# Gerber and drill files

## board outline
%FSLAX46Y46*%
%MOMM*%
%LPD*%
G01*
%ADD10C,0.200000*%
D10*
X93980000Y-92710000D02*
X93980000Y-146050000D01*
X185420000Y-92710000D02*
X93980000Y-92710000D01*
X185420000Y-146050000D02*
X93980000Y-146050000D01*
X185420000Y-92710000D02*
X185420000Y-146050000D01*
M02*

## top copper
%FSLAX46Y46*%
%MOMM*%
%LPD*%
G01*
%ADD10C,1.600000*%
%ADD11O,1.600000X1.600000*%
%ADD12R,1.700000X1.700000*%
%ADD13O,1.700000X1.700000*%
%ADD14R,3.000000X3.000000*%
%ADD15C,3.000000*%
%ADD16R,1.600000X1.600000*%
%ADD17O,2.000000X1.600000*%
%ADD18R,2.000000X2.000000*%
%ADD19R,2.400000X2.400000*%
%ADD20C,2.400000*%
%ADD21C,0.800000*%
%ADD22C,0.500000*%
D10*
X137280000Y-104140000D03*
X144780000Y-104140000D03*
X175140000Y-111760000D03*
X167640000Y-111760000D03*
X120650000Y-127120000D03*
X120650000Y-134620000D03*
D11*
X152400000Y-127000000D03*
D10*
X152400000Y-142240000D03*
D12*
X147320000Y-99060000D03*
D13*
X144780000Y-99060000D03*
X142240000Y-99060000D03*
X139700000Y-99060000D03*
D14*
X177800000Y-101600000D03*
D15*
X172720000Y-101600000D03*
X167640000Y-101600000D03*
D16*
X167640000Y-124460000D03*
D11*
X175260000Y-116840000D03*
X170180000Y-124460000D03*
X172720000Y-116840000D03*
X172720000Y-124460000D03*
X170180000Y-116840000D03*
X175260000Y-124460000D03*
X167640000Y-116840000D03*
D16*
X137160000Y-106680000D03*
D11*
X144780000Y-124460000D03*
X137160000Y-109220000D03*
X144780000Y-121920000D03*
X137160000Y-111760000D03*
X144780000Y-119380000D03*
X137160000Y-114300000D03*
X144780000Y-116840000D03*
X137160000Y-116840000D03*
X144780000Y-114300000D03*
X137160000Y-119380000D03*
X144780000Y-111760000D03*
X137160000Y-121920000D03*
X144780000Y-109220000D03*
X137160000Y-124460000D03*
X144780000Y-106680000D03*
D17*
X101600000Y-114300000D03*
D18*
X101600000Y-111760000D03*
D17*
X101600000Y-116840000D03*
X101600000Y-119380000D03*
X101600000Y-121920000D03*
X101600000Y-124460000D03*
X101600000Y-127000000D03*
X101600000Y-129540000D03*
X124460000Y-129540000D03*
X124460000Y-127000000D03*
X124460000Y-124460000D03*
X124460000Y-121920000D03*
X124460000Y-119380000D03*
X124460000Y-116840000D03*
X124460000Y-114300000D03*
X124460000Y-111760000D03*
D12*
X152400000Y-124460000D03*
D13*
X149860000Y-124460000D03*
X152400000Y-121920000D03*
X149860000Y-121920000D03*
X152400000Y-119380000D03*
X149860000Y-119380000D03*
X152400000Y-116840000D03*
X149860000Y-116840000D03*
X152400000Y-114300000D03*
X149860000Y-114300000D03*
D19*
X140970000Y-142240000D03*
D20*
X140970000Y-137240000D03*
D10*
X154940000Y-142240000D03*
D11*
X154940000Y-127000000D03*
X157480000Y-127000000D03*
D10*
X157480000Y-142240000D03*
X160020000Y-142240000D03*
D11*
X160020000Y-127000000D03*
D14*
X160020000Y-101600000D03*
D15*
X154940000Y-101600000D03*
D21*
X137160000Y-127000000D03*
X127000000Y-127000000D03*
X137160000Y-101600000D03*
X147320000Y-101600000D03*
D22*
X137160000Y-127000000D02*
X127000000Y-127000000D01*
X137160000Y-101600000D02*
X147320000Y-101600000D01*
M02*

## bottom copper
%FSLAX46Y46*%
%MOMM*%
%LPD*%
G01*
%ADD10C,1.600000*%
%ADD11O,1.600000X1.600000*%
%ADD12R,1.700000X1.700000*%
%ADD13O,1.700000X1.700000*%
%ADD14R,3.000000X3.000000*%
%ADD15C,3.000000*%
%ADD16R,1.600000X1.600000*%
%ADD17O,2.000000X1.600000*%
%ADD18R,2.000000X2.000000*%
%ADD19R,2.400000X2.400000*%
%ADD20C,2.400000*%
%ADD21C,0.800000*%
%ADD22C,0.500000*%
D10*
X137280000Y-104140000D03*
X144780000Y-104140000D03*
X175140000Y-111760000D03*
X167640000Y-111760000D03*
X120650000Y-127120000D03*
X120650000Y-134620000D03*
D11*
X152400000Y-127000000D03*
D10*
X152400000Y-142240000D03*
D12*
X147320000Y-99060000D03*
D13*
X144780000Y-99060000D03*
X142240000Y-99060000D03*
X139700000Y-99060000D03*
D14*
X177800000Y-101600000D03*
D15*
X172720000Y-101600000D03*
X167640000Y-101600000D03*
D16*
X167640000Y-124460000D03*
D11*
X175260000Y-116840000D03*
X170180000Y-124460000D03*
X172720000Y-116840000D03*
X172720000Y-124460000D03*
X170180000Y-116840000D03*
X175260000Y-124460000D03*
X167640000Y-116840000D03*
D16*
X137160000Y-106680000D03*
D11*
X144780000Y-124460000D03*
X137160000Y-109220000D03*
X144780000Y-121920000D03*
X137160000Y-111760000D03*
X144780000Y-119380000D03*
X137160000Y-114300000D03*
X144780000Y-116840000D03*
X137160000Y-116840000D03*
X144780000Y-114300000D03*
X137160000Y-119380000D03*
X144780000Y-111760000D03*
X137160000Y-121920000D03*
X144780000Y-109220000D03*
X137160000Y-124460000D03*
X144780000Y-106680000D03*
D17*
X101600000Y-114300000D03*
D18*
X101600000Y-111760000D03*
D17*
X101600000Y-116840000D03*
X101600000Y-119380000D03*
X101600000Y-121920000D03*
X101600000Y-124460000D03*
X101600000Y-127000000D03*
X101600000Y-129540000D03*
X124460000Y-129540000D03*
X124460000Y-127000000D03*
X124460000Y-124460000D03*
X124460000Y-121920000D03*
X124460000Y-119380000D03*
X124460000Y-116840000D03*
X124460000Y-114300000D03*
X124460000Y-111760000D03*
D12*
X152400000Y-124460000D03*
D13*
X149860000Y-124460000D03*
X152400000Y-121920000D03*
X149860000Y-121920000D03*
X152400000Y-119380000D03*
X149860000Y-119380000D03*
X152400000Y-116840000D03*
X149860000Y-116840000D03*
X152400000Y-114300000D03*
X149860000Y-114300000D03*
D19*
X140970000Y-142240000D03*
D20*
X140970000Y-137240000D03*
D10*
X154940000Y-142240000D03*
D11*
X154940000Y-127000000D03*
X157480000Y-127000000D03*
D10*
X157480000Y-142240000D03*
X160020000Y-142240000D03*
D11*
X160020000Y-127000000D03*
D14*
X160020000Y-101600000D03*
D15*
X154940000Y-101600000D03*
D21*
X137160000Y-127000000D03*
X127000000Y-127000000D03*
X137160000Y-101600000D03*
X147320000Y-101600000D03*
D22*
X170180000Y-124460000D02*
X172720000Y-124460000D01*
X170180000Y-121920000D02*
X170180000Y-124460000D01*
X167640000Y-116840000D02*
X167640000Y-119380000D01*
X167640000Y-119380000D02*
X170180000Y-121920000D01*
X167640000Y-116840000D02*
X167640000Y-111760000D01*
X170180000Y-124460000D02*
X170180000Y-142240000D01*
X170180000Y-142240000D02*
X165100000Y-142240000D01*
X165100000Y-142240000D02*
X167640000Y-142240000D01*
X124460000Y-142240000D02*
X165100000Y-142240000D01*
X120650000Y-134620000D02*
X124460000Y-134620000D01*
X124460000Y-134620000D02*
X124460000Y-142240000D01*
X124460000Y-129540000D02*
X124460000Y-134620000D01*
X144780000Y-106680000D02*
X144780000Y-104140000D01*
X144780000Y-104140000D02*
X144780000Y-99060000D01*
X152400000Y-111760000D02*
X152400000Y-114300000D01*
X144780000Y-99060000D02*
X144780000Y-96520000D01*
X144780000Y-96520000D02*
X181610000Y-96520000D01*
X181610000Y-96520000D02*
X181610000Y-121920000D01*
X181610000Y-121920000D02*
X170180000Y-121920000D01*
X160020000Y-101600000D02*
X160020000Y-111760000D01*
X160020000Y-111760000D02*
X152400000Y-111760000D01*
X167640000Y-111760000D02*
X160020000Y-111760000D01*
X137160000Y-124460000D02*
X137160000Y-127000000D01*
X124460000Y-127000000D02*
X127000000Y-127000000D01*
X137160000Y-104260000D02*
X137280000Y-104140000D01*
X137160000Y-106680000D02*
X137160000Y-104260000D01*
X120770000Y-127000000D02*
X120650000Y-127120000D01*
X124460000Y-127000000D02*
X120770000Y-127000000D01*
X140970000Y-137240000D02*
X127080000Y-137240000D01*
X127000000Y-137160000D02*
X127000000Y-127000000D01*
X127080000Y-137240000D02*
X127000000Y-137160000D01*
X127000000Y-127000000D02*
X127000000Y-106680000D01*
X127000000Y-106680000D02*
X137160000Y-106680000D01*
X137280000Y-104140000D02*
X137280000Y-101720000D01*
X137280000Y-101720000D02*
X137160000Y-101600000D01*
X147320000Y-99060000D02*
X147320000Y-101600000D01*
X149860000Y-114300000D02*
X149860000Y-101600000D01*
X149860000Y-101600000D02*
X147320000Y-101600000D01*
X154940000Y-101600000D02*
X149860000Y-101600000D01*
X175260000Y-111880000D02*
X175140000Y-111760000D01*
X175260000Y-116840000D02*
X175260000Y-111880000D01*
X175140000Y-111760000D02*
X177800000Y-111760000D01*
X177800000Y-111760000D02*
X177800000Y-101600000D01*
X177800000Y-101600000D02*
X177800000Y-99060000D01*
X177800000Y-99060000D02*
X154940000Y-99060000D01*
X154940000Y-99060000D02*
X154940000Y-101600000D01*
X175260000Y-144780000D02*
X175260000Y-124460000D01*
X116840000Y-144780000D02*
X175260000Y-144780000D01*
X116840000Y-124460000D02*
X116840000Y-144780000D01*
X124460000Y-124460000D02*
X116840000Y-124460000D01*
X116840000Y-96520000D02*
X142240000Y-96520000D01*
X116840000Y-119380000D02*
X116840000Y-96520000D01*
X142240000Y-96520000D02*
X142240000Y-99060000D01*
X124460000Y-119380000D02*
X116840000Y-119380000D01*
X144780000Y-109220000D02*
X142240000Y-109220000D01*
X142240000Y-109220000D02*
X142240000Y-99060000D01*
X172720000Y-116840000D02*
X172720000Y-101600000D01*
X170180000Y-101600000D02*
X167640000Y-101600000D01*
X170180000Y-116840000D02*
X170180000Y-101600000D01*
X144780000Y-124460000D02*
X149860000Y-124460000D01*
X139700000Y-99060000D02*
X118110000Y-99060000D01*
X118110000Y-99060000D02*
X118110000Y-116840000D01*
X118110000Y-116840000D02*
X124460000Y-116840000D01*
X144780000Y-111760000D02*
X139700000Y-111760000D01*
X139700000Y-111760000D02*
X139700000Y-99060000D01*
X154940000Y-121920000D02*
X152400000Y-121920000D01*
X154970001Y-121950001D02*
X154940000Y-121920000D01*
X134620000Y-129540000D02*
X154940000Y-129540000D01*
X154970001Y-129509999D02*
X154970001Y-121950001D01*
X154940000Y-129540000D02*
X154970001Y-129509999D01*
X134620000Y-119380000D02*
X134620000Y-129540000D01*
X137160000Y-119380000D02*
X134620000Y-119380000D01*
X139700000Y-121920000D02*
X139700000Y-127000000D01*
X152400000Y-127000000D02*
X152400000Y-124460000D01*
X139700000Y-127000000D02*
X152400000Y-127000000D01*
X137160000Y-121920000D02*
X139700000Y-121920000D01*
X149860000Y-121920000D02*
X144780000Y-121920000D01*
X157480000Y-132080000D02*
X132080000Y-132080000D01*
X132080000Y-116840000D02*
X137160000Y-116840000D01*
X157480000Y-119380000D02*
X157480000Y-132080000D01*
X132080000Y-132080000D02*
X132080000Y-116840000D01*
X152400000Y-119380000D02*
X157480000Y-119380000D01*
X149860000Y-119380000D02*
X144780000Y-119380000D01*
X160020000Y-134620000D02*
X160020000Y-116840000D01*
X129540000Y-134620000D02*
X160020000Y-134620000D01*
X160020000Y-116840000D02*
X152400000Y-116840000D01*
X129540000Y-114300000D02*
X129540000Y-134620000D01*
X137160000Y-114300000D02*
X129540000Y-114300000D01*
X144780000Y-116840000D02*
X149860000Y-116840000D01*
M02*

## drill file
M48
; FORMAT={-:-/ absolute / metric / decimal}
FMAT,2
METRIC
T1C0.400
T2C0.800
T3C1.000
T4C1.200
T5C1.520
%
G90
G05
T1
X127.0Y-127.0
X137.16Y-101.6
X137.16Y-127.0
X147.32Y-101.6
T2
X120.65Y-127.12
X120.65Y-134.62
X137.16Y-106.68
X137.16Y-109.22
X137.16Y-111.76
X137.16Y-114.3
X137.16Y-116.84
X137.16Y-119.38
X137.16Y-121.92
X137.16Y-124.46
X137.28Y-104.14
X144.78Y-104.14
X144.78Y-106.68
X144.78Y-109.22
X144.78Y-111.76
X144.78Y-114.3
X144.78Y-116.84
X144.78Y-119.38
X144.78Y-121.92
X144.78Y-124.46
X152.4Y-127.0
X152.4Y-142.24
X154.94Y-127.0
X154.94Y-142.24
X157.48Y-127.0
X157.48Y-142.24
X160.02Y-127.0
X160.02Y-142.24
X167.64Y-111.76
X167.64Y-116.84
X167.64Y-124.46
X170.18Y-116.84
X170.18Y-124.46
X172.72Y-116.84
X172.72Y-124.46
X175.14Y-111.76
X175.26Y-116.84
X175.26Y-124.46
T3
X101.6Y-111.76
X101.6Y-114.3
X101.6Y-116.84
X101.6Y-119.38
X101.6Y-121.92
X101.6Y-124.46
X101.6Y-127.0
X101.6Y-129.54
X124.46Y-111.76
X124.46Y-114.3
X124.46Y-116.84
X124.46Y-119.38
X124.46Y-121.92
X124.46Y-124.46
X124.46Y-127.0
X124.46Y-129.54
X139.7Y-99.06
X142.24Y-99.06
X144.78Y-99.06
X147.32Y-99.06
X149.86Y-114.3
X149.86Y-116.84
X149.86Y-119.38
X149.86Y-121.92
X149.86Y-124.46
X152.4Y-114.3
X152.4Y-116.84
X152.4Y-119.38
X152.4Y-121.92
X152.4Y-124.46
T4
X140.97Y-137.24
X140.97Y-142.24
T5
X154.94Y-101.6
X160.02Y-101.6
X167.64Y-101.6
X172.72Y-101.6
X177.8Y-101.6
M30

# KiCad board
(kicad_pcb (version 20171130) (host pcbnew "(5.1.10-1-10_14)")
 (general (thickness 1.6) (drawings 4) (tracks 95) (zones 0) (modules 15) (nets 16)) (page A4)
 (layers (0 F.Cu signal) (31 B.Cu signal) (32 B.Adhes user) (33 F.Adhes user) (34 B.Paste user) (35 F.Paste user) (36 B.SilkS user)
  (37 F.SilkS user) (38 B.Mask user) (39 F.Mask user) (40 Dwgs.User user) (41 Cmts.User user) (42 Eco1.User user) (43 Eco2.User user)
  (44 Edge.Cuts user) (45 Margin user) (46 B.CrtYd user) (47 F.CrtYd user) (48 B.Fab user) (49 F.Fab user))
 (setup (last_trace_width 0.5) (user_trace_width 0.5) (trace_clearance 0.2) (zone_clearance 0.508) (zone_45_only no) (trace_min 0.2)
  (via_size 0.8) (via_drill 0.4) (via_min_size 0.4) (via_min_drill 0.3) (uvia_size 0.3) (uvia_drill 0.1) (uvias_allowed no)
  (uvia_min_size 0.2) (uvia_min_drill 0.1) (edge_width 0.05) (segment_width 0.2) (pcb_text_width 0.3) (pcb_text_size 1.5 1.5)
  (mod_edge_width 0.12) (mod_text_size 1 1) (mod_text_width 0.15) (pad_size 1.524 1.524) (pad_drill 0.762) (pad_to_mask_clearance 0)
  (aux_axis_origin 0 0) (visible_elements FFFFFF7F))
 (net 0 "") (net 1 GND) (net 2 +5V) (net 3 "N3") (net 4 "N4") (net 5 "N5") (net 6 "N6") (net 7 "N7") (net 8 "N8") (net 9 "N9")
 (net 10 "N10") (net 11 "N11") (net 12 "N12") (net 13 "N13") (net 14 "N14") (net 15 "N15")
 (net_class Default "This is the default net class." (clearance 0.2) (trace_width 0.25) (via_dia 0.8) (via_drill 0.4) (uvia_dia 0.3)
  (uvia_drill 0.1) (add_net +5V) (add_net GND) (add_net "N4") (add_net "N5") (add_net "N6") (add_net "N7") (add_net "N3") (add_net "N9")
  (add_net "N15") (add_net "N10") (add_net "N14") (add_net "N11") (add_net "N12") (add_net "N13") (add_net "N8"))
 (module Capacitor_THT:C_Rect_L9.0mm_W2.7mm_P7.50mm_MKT (layer F.Cu) (at 144.78 104.14 180)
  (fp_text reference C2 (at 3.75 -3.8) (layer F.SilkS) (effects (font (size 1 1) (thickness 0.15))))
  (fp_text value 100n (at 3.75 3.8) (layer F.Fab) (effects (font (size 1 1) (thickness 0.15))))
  (pad 2 thru_hole circle (at 7.5 0 180) (size 1.6 1.6) (drill 0.8) (layers *.Cu *.Mask) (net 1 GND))
  (pad 1 thru_hole circle (at 0 0 180) (size 1.6 1.6) (drill 0.8) (layers *.Cu *.Mask) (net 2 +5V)))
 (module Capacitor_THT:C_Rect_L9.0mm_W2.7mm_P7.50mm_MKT (layer F.Cu) (at 167.64 111.76)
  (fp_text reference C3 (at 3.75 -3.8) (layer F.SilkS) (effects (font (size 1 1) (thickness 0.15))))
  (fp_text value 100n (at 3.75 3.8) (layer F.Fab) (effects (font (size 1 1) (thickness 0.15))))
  (pad 2 thru_hole circle (at 7.5 0) (size 1.6 1.6) (drill 0.8) (layers *.Cu *.Mask) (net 1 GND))
  (pad 1 thru_hole circle (at 0 0) (size 1.6 1.6) (drill 0.8) (layers *.Cu *.Mask) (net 2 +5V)))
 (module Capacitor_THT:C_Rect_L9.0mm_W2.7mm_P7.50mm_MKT (layer F.Cu) (at 120.65 134.62 90)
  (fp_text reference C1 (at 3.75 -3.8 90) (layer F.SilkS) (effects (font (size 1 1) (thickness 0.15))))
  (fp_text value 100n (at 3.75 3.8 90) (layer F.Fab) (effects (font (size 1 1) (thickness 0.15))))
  (pad 2 thru_hole circle (at 7.5 0 90) (size 1.6 1.6) (drill 0.8) (layers *.Cu *.Mask) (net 1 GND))
  (pad 1 thru_hole circle (at 0 0 90) (size 1.6 1.6) (drill 0.8) (layers *.Cu *.Mask) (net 2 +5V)))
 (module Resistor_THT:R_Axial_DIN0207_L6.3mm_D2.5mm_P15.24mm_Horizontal (layer F.Cu) (at 152.4 142.24 90)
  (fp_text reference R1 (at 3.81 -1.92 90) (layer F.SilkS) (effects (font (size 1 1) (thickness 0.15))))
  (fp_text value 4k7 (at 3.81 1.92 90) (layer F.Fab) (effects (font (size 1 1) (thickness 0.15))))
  (pad 2 thru_hole oval (at 15.24 0 90) (size 1.6 1.6) (drill 0.8) (layers *.Cu *.Mask) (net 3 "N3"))
  (pad 1 thru_hole circle (at 0 0 90) (size 1.6 1.6) (drill 0.8) (layers *.Cu *.Mask) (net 2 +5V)))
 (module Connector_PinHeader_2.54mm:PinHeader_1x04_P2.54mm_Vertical (layer F.Cu) (at 147.32 99.06 270)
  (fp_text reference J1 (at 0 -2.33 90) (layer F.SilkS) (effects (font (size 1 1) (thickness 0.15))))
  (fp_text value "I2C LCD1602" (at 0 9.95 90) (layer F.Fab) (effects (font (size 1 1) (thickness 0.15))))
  (pad 1 thru_hole rect (at 0 0 270) (size 1.7 1.7) (drill 1) (layers *.Cu *.Mask) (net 1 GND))
  (pad 2 thru_hole oval (at 0 2.54 270) (size 1.7 1.7) (drill 1) (layers *.Cu *.Mask) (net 2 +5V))
  (pad 3 thru_hole oval (at 0 5.08 270) (size 1.7 1.7) (drill 1) (layers *.Cu *.Mask) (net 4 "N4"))
  (pad 4 thru_hole oval (at 0 7.62 270) (size 1.7 1.7) (drill 1) (layers *.Cu *.Mask) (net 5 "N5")))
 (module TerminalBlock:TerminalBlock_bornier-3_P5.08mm (layer F.Cu) (at 177.8 101.6 180)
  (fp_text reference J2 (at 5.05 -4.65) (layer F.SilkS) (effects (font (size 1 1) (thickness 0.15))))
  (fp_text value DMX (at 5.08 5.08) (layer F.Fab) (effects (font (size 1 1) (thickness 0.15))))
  (pad 1 thru_hole rect (at 0 0 180) (size 3 3) (drill 1.52) (layers *.Cu *.Mask) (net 1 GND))
  (pad 2 thru_hole circle (at 5.08 0 180) (size 3 3) (drill 1.52) (layers *.Cu *.Mask) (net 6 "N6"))
  (pad 3 thru_hole circle (at 10.16 0 180) (size 3 3) (drill 1.52) (layers *.Cu *.Mask) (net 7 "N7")))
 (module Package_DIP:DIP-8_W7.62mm (layer F.Cu) (at 167.64 124.46 90)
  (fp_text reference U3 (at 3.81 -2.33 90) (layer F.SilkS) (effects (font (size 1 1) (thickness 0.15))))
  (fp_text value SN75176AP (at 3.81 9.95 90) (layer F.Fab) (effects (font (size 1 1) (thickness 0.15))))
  (pad 1 thru_hole rect (at 0 0 90) (size 1.6 1.6) (drill 0.8) (layers *.Cu *.Mask))
  (pad 5 thru_hole oval (at 7.62 7.62 90) (size 1.6 1.6) (drill 0.8) (layers *.Cu *.Mask) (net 1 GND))
  (pad 2 thru_hole oval (at 0 2.54 90) (size 1.6 1.6) (drill 0.8) (layers *.Cu *.Mask) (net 2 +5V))
  (pad 6 thru_hole oval (at 7.62 5.08 90) (size 1.6 1.6) (drill 0.8) (layers *.Cu *.Mask) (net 6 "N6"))
  (pad 3 thru_hole oval (at 0 5.08 90) (size 1.6 1.6) (drill 0.8) (layers *.Cu *.Mask) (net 2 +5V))
  (pad 7 thru_hole oval (at 7.62 2.54 90) (size 1.6 1.6) (drill 0.8) (layers *.Cu *.Mask) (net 7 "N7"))
  (pad 4 thru_hole oval (at 0 7.62 90) (size 1.6 1.6) (drill 0.8) (layers *.Cu *.Mask) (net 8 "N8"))
  (pad 8 thru_hole oval (at 7.62 0 90) (size 1.6 1.6) (drill 0.8) (layers *.Cu *.Mask) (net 2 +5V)))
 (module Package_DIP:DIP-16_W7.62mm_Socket (layer F.Cu) (at 137.16 106.68)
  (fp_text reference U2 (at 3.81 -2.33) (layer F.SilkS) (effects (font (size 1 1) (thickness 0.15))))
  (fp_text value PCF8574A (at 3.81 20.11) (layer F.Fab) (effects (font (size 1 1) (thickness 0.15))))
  (pad 1 thru_hole rect (at 0 0) (size 1.6 1.6) (drill 0.8) (layers *.Cu *.Mask) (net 1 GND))
  (pad 9 thru_hole oval (at 7.62 17.78) (size 1.6 1.6) (drill 0.8) (layers *.Cu *.Mask) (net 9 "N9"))
  (pad 2 thru_hole oval (at 0 2.54) (size 1.6 1.6) (drill 0.8) (layers *.Cu *.Mask))
  (pad 10 thru_hole oval (at 7.62 15.24) (size 1.6 1.6) (drill 0.8) (layers *.Cu *.Mask) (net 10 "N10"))
  (pad 3 thru_hole oval (at 0 5.08) (size 1.6 1.6) (drill 0.8) (layers *.Cu *.Mask))
  (pad 11 thru_hole oval (at 7.62 12.7) (size 1.6 1.6) (drill 0.8) (layers *.Cu *.Mask) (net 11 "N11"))
  (pad 4 thru_hole oval (at 0 7.62) (size 1.6 1.6) (drill 0.8) (layers *.Cu *.Mask) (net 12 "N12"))
  (pad 12 thru_hole oval (at 7.62 10.16) (size 1.6 1.6) (drill 0.8) (layers *.Cu *.Mask) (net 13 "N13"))
  (pad 5 thru_hole oval (at 0 10.16) (size 1.6 1.6) (drill 0.8) (layers *.Cu *.Mask) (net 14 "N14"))
  (pad 13 thru_hole oval (at 7.62 7.62) (size 1.6 1.6) (drill 0.8) (layers *.Cu *.Mask))
  (pad 6 thru_hole oval (at 0 12.7) (size 1.6 1.6) (drill 0.8) (layers *.Cu *.Mask) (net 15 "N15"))
  (pad 14 thru_hole oval (at 7.62 5.08) (size 1.6 1.6) (drill 0.8) (layers *.Cu *.Mask) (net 5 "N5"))
  (pad 7 thru_hole oval (at 0 15.24) (size 1.6 1.6) (drill 0.8) (layers *.Cu *.Mask) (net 3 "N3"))
  (pad 15 thru_hole oval (at 7.62 2.54) (size 1.6 1.6) (drill 0.8) (layers *.Cu *.Mask) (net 4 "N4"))
  (pad 8 thru_hole oval (at 0 17.78) (size 1.6 1.6) (drill 0.8) (layers *.Cu *.Mask) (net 1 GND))
  (pad 16 thru_hole oval (at 7.62 0) (size 1.6 1.6) (drill 0.8) (layers *.Cu *.Mask) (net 2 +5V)))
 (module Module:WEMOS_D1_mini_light (layer F.Cu) (at 101.6 111.76)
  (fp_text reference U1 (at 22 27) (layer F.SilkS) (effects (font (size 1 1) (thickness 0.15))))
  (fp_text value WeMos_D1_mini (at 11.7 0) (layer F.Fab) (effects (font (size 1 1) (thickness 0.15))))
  (pad 2 thru_hole oval (at 0 2.54) (size 2 1.6) (drill 1) (layers *.Cu *.Mask))
  (pad 1 thru_hole rect (at 0 0) (size 2 2) (drill 1) (layers *.Cu *.Mask))
  (pad 3 thru_hole oval (at 0 5.08) (size 2 1.6) (drill 1) (layers *.Cu *.Mask))
  (pad 4 thru_hole oval (at 0 7.62) (size 2 1.6) (drill 1) (layers *.Cu *.Mask))
  (pad 5 thru_hole oval (at 0 10.16) (size 2 1.6) (drill 1) (layers *.Cu *.Mask))
  (pad 6 thru_hole oval (at 0 12.7) (size 2 1.6) (drill 1) (layers *.Cu *.Mask))
  (pad 7 thru_hole oval (at 0 15.24) (size 2 1.6) (drill 1) (layers *.Cu *.Mask))
  (pad 8 thru_hole oval (at 0 17.78) (size 2 1.6) (drill 1) (layers *.Cu *.Mask))
  (pad 9 thru_hole oval (at 22.86 17.78) (size 2 1.6) (drill 1) (layers *.Cu *.Mask) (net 2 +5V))
  (pad 10 thru_hole oval (at 22.86 15.24) (size 2 1.6) (drill 1) (layers *.Cu *.Mask) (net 1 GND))
  (pad 11 thru_hole oval (at 22.86 12.7) (size 2 1.6) (drill 1) (layers *.Cu *.Mask) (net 8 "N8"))
  (pad 12 thru_hole oval (at 22.86 10.16) (size 2 1.6) (drill 1) (layers *.Cu *.Mask))
  (pad 13 thru_hole oval (at 22.86 7.62) (size 2 1.6) (drill 1) (layers *.Cu *.Mask) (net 4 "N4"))
  (pad 14 thru_hole oval (at 22.86 5.08) (size 2 1.6) (drill 1) (layers *.Cu *.Mask) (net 5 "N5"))
  (pad 15 thru_hole oval (at 22.86 2.54) (size 2 1.6) (drill 1) (layers *.Cu *.Mask))
  (pad 16 thru_hole oval (at 22.86 0) (size 2 1.6) (drill 1) (layers *.Cu *.Mask)))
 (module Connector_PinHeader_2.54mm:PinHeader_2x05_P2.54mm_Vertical (layer F.Cu) (at 152.4 124.46 180)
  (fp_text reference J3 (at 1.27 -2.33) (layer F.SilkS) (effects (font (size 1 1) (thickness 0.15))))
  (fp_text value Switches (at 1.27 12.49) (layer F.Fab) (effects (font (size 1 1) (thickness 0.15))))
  (pad 1 thru_hole rect (at 0 0 180) (size 1.7 1.7) (drill 1) (layers *.Cu *.Mask) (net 3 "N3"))
  (pad 2 thru_hole oval (at 2.54 0 180) (size 1.7 1.7) (drill 1) (layers *.Cu *.Mask) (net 9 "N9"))
  (pad 3 thru_hole oval (at 0 2.54 180) (size 1.7 1.7) (drill 1) (layers *.Cu *.Mask) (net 15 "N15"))
  (pad 4 thru_hole oval (at 2.54 2.54 180) (size 1.7 1.7) (drill 1) (layers *.Cu *.Mask) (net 10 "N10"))
  (pad 5 thru_hole oval (at 0 5.08 180) (size 1.7 1.7) (drill 1) (layers *.Cu *.Mask) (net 14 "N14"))
  (pad 6 thru_hole oval (at 2.54 5.08 180) (size 1.7 1.7) (drill 1) (layers *.Cu *.Mask) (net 11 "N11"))
  (pad 7 thru_hole oval (at 0 7.62 180) (size 1.7 1.7) (drill 1) (layers *.Cu *.Mask) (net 12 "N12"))
  (pad 8 thru_hole oval (at 2.54 7.62 180) (size 1.7 1.7) (drill 1) (layers *.Cu *.Mask) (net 13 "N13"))
  (pad 9 thru_hole oval (at 0 10.16 180) (size 1.7 1.7) (drill 1) (layers *.Cu *.Mask) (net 2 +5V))
  (pad 10 thru_hole oval (at 2.54 10.16 180) (size 1.7 1.7) (drill 1) (layers *.Cu *.Mask) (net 1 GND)))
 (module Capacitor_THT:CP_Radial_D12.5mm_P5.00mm (layer F.Cu) (at 140.97 142.24 90)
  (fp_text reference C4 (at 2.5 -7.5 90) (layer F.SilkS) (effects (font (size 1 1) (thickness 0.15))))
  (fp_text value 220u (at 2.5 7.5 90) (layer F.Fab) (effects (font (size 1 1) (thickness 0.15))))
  (pad 1 thru_hole rect (at 0 0 90) (size 2.4 2.4) (drill 1.2) (layers *.Cu *.Mask) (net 2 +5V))
  (pad 2 thru_hole circle (at 5 0 90) (size 2.4 2.4) (drill 1.2) (layers *.Cu *.Mask) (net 1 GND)))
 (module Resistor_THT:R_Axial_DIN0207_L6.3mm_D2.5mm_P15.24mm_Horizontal (layer F.Cu) (at 154.94 142.24 90)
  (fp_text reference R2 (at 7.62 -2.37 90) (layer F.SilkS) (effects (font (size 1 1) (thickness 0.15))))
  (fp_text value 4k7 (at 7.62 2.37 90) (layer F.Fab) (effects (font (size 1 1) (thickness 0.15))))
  (pad 1 thru_hole circle (at 0 0 90) (size 1.6 1.6) (drill 0.8) (layers *.Cu *.Mask) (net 2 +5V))
  (pad 2 thru_hole oval (at 15.24 0 90) (size 1.6 1.6) (drill 0.8) (layers *.Cu *.Mask) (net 15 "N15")))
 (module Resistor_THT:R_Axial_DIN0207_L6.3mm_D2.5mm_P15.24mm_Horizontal (layer F.Cu) (at 157.48 142.24 90)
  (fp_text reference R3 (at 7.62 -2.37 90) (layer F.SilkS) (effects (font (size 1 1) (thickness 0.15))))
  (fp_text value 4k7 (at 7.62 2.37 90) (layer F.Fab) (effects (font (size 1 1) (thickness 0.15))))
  (pad 2 thru_hole oval (at 15.24 0 90) (size 1.6 1.6) (drill 0.8) (layers *.Cu *.Mask) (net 14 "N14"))
  (pad 1 thru_hole circle (at 0 0 90) (size 1.6 1.6) (drill 0.8) (layers *.Cu *.Mask) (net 2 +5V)))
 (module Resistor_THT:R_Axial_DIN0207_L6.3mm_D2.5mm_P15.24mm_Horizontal (layer F.Cu) (at 160.02 142.24 90)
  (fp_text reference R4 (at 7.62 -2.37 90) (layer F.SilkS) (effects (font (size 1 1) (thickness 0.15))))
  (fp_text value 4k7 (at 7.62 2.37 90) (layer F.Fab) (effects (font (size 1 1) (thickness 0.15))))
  (pad 1 thru_hole circle (at 0 0 90) (size 1.6 1.6) (drill 0.8) (layers *.Cu *.Mask) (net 2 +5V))
  (pad 2 thru_hole oval (at 15.24 0 90) (size 1.6 1.6) (drill 0.8) (layers *.Cu *.Mask) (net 12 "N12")))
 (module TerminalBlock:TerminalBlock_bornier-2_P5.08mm (layer F.Cu) (at 160.02 101.6 180)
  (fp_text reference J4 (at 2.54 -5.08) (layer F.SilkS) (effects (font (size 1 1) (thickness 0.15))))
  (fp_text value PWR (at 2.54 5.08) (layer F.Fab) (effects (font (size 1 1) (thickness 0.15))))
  (pad 1 thru_hole rect (at 0 0 180) (size 3 3) (drill 1.52) (layers *.Cu *.Mask) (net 2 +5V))
  (pad 2 thru_hole circle (at 5.08 0 180) (size 3 3) (drill 1.52) (layers *.Cu *.Mask) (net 1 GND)))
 (gr_line (start 93.98 92.71) (end 93.98 146.05) (layer Edge.Cuts) (width 0.2))
 (gr_line (start 185.42 92.71) (end 93.98 92.71) (layer Edge.Cuts) (width 0.2))
 (gr_line (start 185.42 146.05) (end 93.98 146.05) (layer Edge.Cuts) (width 0.2))
 (gr_line (start 185.42 92.71) (end 185.42 146.05) (layer Edge.Cuts) (width 0.2))
 (segment (start 170.18 124.46) (end 172.72 124.46) (width 0.5) (layer B.Cu) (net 2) (status 30))
 (segment (start 170.18 121.92) (end 170.18 124.46) (width 0.5) (layer B.Cu) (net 2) (status 20))
 (segment (start 167.64 116.84) (end 167.64 119.38) (width 0.5) (layer B.Cu) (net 2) (status 10))
 (segment (start 167.64 119.38) (end 170.18 121.92) (width 0.5) (layer B.Cu) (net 2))
 (segment (start 167.64 116.84) (end 167.64 111.76) (width 0.5) (layer B.Cu) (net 2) (status 30))
 (segment (start 170.18 124.46) (end 170.18 142.24) (width 0.5) (layer B.Cu) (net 2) (status 10))
 (segment (start 170.18 142.24) (end 165.1 142.24) (width 0.5) (layer B.Cu) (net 2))
 (segment (start 165.1 142.24) (end 167.64 142.24) (width 0.5) (layer B.Cu) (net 2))
 (segment (start 124.46 142.24) (end 165.1 142.24) (width 0.5) (layer B.Cu) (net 2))
 (segment (start 120.65 134.62) (end 124.46 134.62) (width 0.5) (layer B.Cu) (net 2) (status 10))
 (segment (start 124.46 134.62) (end 124.46 142.24) (width 0.5) (layer B.Cu) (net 2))
 (segment (start 124.46 129.54) (end 124.46 134.62) (width 0.5) (layer B.Cu) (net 2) (status 10))
 (segment (start 144.78 106.68) (end 144.78 104.14) (width 0.5) (layer B.Cu) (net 2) (status 30))
 (segment (start 144.78 104.14) (end 144.78 99.06) (width 0.5) (layer B.Cu) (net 2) (status 30))
 (segment (start 152.4 111.76) (end 152.4 114.3) (width 0.5) (layer B.Cu) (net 2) (status 20))
 (segment (start 144.78 99.06) (end 144.78 96.52) (width 0.5) (layer B.Cu) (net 2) (status 10))
 (segment (start 144.78 96.52) (end 181.61 96.52) (width 0.5) (layer B.Cu) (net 2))
 (segment (start 181.61 96.52) (end 181.61 121.92) (width 0.5) (layer B.Cu) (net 2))
 (segment (start 181.61 121.92) (end 170.18 121.92) (width 0.5) (layer B.Cu) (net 2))
 (segment (start 160.02 101.6) (end 160.02 111.76) (width 0.5) (layer B.Cu) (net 2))
 (segment (start 160.02 111.76) (end 152.4 111.76) (width 0.5) (layer B.Cu) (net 2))
 (segment (start 167.64 111.76) (end 160.02 111.76) (width 0.5) (layer B.Cu) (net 2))
 (segment (start 137.16 124.46) (end 137.16 127) (width 0.5) (layer B.Cu) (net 1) (status 10))
 (via (at 137.16 127) (size 0.8) (drill 0.4) (layers F.Cu B.Cu) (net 1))
 (via (at 127 127) (size 0.8) (drill 0.4) (layers F.Cu B.Cu) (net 1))
 (segment (start 137.16 127) (end 127 127) (width 0.5) (layer F.Cu) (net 1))
 (segment (start 124.46 127) (end 127 127) (width 0.5) (layer B.Cu) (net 1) (status 10))
 (segment (start 137.16 104.26) (end 137.28 104.14) (width 0.5) (layer B.Cu) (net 1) (status 30))
 (segment (start 137.16 106.68) (end 137.16 104.26) (width 0.5) (layer B.Cu) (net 1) (status 30))
 (segment (start 120.77 127) (end 120.65 127.12) (width 0.5) (layer B.Cu) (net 1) (status 30))
 (segment (start 124.46 127) (end 120.77 127) (width 0.5) (layer B.Cu) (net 1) (status 30))
 (segment (start 140.97 137.24) (end 127.08 137.24) (width 0.5) (layer B.Cu) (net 1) (status 10))
 (segment (start 127 137.16) (end 127 127) (width 0.5) (layer B.Cu) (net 1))
 (segment (start 127.08 137.24) (end 127 137.16) (width 0.5) (layer B.Cu) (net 1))
 (segment (start 127 127) (end 127 106.68) (width 0.5) (layer B.Cu) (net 1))
 (segment (start 127 106.68) (end 137.16 106.68) (width 0.5) (layer B.Cu) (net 1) (status 20))
 (segment (start 137.28 104.14) (end 137.28 101.72) (width 0.5) (layer B.Cu) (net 1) (status 10))
 (via (at 137.16 101.6) (size 0.8) (drill 0.4) (layers F.Cu B.Cu) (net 1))
 (segment (start 137.28 101.72) (end 137.16 101.6) (width 0.5) (layer B.Cu) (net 1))
 (segment (start 137.16 101.6) (end 147.32 101.6) (width 0.5) (layer F.Cu) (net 1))
 (via (at 147.32 101.6) (size 0.8) (drill 0.4) (layers F.Cu B.Cu) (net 1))
 (segment (start 147.32 99.06) (end 147.32 101.6) (width 0.5) (layer B.Cu) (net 1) (status 10))
 (segment (start 149.86 114.3) (end 149.86 101.6) (width 0.5) (layer B.Cu) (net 1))
 (segment (start 149.86 101.6) (end 147.32 101.6) (width 0.5) (layer B.Cu) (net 1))
 (segment (start 154.94 101.6) (end 149.86 101.6) (width 0.5) (layer B.Cu) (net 1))
 (segment (start 175.26 111.88) (end 175.14 111.76) (width 0.5) (layer B.Cu) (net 1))
 (segment (start 175.26 116.84) (end 175.26 111.88) (width 0.5) (layer B.Cu) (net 1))
 (segment (start 175.14 111.76) (end 177.8 111.76) (width 0.5) (layer B.Cu) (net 1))
 (segment (start 177.8 111.76) (end 177.8 101.6) (width 0.5) (layer B.Cu) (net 1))
 (segment (start 177.8 101.6) (end 177.8 99.06) (width 0.5) (layer B.Cu) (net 1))
 (segment (start 177.8 99.06) (end 154.94 99.06) (width 0.5) (layer B.Cu) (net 1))
 (segment (start 154.94 99.06) (end 154.94 101.6) (width 0.5) (layer B.Cu) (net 1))
 (segment (start 175.26 144.78) (end 175.26 124.46) (width 0.5) (layer B.Cu) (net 8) (status 20))
 (segment (start 116.84 144.78) (end 175.26 144.78) (width 0.5) (layer B.Cu) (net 8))
 (segment (start 116.84 124.46) (end 116.84 144.78) (width 0.5) (layer B.Cu) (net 8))
 (segment (start 124.46 124.46) (end 116.84 124.46) (width 0.5) (layer B.Cu) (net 8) (status 10))
 (segment (start 116.84 96.52) (end 142.24 96.52) (width 0.5) (layer B.Cu) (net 4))
 (segment (start 116.84 119.38) (end 116.84 96.52) (width 0.5) (layer B.Cu) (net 4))
 (segment (start 142.24 96.52) (end 142.24 99.06) (width 0.5) (layer B.Cu) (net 4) (status 20))
 (segment (start 124.46 119.38) (end 116.84 119.38) (width 0.5) (layer B.Cu) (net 4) (status 10))
 (segment (start 144.78 109.22) (end 142.24 109.22) (width 0.5) (layer B.Cu) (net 4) (status 10))
 (segment (start 142.24 109.22) (end 142.24 99.06) (width 0.5) (layer B.Cu) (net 4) (status 20))
 (segment (start 172.72 116.84) (end 172.72 101.6) (width 0.5) (layer B.Cu) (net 6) (status 30))
 (segment (start 170.18 101.6) (end 167.64 101.6) (width 0.5) (layer B.Cu) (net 7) (status 20))
 (segment (start 170.18 116.84) (end 170.18 101.6) (width 0.5) (layer B.Cu) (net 7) (status 10))
 (segment (start 144.78 124.46) (end 149.86 124.46) (width 0.5) (layer B.Cu) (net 9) (status 30))
 (segment (start 139.7 99.06) (end 118.11 99.06) (width 0.5) (layer B.Cu) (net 5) (status 10))
 (segment (start 118.11 99.06) (end 118.11 116.84) (width 0.5) (layer B.Cu) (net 5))
 (segment (start 118.11 116.84) (end 124.46 116.84) (width 0.5) (layer B.Cu) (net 5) (status 20))
 (segment (start 144.78 111.76) (end 139.7 111.76) (width 0.5) (layer B.Cu) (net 5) (status 10))
 (segment (start 139.7 111.76) (end 139.7 99.06) (width 0.5) (layer B.Cu) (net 5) (status 20))
 (segment (start 154.94 121.92) (end 152.4 121.92) (width 0.5) (layer B.Cu) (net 15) (status 20))
 (segment (start 154.970001 121.950001) (end 154.94 121.92) (width 0.5) (layer B.Cu) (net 15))
 (segment (start 134.62 129.54) (end 154.94 129.54) (width 0.5) (layer B.Cu) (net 15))
 (segment (start 154.970001 129.509999) (end 154.970001 121.950001) (width 0.5) (layer B.Cu) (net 15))
 (segment (start 154.94 129.54) (end 154.970001 129.509999) (width 0.5) (layer B.Cu) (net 15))
 (segment (start 134.62 119.38) (end 134.62 129.54) (width 0.5) (layer B.Cu) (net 15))
 (segment (start 137.16 119.38) (end 134.62 119.38) (width 0.5) (layer B.Cu) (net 15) (status 10))
 (segment (start 139.7 121.92) (end 139.7 127) (width 0.5) (layer B.Cu) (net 3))
 (segment (start 152.4 127) (end 152.4 124.46) (width 0.5) (layer B.Cu) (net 3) (status 30))
 (segment (start 139.7 127) (end 152.4 127) (width 0.5) (layer B.Cu) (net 3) (status 20))
 (segment (start 137.16 121.92) (end 139.7 121.92) (width 0.5) (layer B.Cu) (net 3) (status 10))
 (segment (start 149.86 121.92) (end 144.78 121.92) (width 0.5) (layer B.Cu) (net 10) (status 30))
 (segment (start 157.48 132.08) (end 132.08 132.08) (width 0.5) (layer B.Cu) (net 14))
 (segment (start 132.08 116.84) (end 137.16 116.84) (width 0.5) (layer B.Cu) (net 14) (status 20))
 (segment (start 157.48 119.38) (end 157.48 132.08) (width 0.5) (layer B.Cu) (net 14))
 (segment (start 132.08 132.08) (end 132.08 116.84) (width 0.5) (layer B.Cu) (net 14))
 (segment (start 152.4 119.38) (end 157.48 119.38) (width 0.5) (layer B.Cu) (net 14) (status 10))
 (segment (start 149.86 119.38) (end 144.78 119.38) (width 0.5) (layer B.Cu) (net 11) (status 30))
 (segment (start 160.02 134.62) (end 160.02 116.84) (width 0.5) (layer B.Cu) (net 12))
 (segment (start 129.54 134.62) (end 160.02 134.62) (width 0.5) (layer B.Cu) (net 12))
 (segment (start 160.02 116.84) (end 152.4 116.84) (width 0.5) (layer B.Cu) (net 12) (status 20))
 (segment (start 129.54 114.3) (end 129.54 134.62) (width 0.5) (layer B.Cu) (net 12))
 (segment (start 137.16 114.3) (end 129.54 114.3) (width 0.5) (layer B.Cu) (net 12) (status 10))
 (segment (start 144.78 116.84) (end 149.86 116.84) (width 0.5) (layer B.Cu) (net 13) (status 30)))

